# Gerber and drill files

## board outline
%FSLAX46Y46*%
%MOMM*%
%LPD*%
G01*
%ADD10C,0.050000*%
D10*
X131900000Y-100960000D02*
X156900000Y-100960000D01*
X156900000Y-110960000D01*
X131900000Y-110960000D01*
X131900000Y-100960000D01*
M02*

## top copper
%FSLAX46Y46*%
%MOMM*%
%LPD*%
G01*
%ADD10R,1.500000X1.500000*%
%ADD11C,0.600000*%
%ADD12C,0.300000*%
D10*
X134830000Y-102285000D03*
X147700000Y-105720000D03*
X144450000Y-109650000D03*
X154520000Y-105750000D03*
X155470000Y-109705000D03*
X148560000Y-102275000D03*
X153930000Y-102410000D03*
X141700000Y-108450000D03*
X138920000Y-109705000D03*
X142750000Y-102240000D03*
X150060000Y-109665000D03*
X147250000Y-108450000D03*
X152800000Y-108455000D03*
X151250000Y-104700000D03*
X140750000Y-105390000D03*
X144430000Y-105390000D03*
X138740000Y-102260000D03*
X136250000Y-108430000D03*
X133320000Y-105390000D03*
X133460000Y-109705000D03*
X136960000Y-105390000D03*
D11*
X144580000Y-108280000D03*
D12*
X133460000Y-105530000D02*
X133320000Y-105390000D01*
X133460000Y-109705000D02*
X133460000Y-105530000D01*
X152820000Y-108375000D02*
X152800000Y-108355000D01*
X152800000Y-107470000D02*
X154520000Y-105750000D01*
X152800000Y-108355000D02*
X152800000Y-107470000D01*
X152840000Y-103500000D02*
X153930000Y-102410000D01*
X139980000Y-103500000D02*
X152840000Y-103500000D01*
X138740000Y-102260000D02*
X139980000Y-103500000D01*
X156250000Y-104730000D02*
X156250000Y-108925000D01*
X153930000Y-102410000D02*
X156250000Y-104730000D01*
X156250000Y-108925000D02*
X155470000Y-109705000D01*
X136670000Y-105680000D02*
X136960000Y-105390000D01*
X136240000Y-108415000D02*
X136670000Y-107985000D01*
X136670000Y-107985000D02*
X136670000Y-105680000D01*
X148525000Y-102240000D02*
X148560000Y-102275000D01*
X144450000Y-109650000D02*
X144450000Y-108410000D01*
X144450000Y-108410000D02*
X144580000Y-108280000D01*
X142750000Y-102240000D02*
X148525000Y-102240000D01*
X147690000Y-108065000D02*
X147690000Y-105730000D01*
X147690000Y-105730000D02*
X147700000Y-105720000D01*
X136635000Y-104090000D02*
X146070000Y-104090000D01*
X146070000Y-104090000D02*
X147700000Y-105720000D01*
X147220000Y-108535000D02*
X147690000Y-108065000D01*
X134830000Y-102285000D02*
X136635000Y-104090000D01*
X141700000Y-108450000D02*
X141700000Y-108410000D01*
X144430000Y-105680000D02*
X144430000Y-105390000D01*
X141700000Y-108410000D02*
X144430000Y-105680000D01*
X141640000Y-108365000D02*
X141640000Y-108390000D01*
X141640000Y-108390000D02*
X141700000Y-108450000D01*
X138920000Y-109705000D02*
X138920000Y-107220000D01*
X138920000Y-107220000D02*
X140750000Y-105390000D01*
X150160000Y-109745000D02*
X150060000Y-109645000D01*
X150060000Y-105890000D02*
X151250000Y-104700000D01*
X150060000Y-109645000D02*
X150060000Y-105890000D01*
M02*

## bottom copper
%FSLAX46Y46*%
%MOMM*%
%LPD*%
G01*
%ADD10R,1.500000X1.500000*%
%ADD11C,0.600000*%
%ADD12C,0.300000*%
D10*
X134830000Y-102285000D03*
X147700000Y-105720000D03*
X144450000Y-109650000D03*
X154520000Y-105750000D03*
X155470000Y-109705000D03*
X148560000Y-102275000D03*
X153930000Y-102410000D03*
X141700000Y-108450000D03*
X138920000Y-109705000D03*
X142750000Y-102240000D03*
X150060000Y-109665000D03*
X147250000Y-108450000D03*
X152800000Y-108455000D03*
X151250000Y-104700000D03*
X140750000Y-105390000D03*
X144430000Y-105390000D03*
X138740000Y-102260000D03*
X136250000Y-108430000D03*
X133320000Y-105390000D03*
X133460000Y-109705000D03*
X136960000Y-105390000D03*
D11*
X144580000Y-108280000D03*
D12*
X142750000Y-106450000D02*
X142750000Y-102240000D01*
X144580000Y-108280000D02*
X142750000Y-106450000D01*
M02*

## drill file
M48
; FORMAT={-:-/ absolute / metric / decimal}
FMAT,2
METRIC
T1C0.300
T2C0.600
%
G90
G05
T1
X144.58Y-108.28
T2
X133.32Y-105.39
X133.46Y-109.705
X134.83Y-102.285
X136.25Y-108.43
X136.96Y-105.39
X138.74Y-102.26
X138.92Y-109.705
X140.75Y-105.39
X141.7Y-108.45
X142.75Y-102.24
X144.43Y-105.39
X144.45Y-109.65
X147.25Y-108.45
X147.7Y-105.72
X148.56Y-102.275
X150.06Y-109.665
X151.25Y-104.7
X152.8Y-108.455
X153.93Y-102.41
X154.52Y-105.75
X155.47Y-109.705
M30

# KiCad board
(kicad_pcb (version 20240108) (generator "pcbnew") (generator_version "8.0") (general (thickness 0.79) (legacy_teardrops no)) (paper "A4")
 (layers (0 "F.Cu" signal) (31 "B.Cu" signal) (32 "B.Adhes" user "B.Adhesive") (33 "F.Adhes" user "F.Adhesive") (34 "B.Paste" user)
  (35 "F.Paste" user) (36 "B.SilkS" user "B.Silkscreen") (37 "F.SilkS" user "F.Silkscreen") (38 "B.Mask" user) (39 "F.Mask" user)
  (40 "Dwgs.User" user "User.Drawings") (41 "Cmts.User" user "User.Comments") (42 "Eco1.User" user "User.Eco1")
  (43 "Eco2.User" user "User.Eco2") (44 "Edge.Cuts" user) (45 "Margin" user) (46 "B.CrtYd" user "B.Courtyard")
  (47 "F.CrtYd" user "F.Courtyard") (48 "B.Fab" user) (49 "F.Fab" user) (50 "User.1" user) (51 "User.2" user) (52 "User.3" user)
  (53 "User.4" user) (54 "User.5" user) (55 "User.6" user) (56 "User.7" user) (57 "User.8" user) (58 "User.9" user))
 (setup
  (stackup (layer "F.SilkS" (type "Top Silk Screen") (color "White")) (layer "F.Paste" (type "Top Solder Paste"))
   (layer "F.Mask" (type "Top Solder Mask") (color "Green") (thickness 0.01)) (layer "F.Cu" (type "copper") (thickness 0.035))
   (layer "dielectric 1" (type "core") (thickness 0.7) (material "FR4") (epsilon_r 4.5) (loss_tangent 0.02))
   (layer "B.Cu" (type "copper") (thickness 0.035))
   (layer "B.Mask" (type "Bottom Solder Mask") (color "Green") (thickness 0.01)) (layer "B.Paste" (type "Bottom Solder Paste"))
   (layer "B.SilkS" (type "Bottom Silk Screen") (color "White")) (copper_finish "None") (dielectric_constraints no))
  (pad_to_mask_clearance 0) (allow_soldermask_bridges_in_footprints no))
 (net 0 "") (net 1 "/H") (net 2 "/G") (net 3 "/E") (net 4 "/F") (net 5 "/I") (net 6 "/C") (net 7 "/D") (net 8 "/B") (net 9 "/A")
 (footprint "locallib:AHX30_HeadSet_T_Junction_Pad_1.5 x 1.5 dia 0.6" (layer "F.Cu") (at 134.83 102.285 180)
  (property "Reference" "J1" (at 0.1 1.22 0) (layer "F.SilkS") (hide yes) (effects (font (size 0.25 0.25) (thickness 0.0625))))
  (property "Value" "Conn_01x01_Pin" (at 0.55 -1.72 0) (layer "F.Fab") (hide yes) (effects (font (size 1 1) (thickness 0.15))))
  (pad "1" thru_hole rect (at 0 0 180) (size 1.5 1.5) (drill 0.6) (layers "*.Cu" "*.Mask") (remove_unused_layers no) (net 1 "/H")))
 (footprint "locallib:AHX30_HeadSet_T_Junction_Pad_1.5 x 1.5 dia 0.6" (layer "F.Cu") (at 147.7 105.72 180)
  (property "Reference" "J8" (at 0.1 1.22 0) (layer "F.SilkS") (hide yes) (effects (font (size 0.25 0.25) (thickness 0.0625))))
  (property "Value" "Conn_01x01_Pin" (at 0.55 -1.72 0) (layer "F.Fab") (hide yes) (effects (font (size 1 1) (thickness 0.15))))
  (pad "1" thru_hole rect (at 0 0 180) (size 1.5 1.5) (drill 0.6) (layers "*.Cu" "*.Mask") (remove_unused_layers no) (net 1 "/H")))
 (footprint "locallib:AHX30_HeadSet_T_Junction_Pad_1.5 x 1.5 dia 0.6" (layer "F.Cu") (at 144.45 109.65)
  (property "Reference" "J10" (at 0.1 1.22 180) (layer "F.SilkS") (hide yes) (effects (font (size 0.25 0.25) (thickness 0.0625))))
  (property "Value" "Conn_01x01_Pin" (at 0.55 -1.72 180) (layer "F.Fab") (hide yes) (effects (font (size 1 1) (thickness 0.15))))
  (pad "1" thru_hole rect (at 0 0) (size 1.5 1.5) (drill 0.6) (layers "*.Cu" "*.Mask") (remove_unused_layers no) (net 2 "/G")))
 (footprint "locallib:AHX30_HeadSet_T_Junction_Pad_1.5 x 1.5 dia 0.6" (layer "F.Cu") (at 154.52 105.75 180)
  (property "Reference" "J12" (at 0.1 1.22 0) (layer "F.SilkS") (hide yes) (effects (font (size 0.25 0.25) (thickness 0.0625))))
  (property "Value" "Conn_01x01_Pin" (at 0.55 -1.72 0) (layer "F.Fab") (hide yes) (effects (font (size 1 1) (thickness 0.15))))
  (pad "1" thru_hole rect (at 0 0 180) (size 1.5 1.5) (drill 0.6) (layers "*.Cu" "*.Mask") (remove_unused_layers no) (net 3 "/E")))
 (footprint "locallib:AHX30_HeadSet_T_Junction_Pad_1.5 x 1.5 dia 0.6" (layer "F.Cu") (at 155.47 109.705)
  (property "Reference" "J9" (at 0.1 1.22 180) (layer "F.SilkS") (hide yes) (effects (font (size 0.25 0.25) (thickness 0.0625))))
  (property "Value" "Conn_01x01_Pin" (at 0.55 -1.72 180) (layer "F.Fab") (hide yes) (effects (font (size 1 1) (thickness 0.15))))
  (pad "1" thru_hole rect (at 0 0) (size 1.5 1.5) (drill 0.6) (layers "*.Cu" "*.Mask") (remove_unused_layers no) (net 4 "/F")))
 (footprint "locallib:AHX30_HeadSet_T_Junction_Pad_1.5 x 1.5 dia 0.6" (layer "F.Cu") (at 148.56 102.275)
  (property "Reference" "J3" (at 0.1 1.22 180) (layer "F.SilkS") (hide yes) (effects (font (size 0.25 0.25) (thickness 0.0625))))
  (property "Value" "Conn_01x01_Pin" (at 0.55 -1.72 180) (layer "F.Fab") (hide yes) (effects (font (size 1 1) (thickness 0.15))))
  (pad "1" thru_hole rect (at 0 0) (size 1.5 1.5) (drill 0.6) (layers "*.Cu" "*.Mask") (remove_unused_layers no) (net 2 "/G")))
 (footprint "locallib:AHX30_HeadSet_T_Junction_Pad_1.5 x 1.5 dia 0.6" (layer "F.Cu") (at 153.93 102.41 180)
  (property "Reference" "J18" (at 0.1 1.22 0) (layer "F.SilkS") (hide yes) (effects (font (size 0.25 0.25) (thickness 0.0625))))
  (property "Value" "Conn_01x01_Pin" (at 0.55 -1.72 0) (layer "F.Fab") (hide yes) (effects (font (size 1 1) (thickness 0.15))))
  (pad "1" thru_hole rect (at 0 0 180) (size 1.5 1.5) (drill 0.6) (layers "*.Cu" "*.Mask") (remove_unused_layers no) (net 4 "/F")))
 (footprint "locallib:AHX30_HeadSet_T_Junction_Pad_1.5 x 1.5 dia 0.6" (layer "F.Cu") (at 141.7 108.45)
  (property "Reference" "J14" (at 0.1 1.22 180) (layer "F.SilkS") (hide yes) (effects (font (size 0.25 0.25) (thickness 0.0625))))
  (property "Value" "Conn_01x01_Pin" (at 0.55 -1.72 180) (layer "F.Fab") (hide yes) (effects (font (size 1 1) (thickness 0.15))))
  (pad "1" thru_hole rect (at 0 0) (size 1.5 1.5) (drill 0.6) (layers "*.Cu" "*.Mask") (remove_unused_layers no) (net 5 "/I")))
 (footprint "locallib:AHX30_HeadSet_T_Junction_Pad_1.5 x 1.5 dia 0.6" (layer "F.Cu") (at 138.92 109.705)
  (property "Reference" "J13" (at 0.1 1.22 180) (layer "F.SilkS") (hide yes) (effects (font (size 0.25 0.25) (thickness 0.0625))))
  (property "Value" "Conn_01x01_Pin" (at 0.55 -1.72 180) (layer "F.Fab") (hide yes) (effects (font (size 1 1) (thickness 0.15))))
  (pad "1" thru_hole rect (at 0 0) (size 1.5 1.5) (drill 0.6) (layers "*.Cu" "*.Mask") (remove_unused_layers no) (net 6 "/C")))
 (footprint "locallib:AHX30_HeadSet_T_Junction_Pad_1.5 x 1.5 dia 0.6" (layer "F.Cu") (at 142.75 102.24 180)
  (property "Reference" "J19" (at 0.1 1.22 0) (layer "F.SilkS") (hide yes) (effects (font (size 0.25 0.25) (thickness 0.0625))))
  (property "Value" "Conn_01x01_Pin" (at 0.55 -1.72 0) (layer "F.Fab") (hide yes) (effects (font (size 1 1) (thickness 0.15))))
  (pad "1" thru_hole rect (at 0 0 180) (size 1.5 1.5) (drill 0.6) (layers "*.Cu" "*.Mask") (remove_unused_layers no) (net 2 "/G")))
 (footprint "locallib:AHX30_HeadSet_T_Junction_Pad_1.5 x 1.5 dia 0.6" (layer "F.Cu") (at 150.06 109.665)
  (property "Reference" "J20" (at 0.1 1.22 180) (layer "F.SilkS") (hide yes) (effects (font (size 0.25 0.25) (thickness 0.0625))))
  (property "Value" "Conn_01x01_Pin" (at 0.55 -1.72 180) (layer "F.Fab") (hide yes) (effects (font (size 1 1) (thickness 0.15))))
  (pad "1" thru_hole rect (at 0 0) (size 1.5 1.5) (drill 0.6) (layers "*.Cu" "*.Mask") (remove_unused_layers no) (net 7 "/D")))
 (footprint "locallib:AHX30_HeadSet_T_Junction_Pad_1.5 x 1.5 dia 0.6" (layer "F.Cu") (at 147.25 108.45)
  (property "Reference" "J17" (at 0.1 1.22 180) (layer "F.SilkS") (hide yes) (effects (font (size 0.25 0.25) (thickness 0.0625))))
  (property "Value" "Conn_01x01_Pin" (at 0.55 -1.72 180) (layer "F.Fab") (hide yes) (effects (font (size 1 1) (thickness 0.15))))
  (pad "1" thru_hole rect (at 0 0) (size 1.5 1.5) (drill 0.6) (layers "*.Cu" "*.Mask") (remove_unused_layers no) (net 1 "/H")))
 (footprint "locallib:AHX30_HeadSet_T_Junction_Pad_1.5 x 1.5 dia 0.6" (layer "F.Cu") (at 152.8 108.455)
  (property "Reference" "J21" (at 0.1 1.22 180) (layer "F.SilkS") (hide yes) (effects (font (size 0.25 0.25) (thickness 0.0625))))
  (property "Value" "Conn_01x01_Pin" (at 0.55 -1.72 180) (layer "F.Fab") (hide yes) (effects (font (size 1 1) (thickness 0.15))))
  (pad "1" thru_hole rect (at 0 0) (size 1.5 1.5) (drill 0.6) (layers "*.Cu" "*.Mask") (remove_unused_layers no) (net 3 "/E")))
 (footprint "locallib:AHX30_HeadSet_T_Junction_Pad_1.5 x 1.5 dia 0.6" (layer "F.Cu") (at 151.25 104.7 180)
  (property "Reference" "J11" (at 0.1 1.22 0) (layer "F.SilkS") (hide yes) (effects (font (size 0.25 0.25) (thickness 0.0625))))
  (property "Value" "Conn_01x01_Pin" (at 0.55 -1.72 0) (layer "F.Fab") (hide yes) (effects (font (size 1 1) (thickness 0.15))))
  (pad "1" thru_hole rect (at 0 0 180) (size 1.5 1.5) (drill 0.6) (layers "*.Cu" "*.Mask") (remove_unused_layers no) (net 7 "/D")))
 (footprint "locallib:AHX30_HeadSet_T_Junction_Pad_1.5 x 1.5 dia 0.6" (layer "F.Cu") (at 140.75 105.39 180)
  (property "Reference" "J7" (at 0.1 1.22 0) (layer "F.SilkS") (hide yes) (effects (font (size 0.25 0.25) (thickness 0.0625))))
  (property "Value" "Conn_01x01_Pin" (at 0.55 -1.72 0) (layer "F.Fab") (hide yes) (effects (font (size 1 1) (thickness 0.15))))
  (pad "1" thru_hole rect (at 0 0 180) (size 1.5 1.5) (drill 0.6) (layers "*.Cu" "*.Mask") (remove_unused_layers no) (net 6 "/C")))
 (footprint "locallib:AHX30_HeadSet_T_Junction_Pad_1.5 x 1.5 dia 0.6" (layer "F.Cu") (at 144.43 105.39 180)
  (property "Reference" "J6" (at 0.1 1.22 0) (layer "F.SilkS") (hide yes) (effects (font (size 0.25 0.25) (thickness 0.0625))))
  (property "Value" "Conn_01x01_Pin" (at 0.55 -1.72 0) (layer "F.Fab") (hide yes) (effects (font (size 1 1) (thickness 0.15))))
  (pad "1" thru_hole rect (at 0 0 180) (size 1.5 1.5) (drill 0.6) (layers "*.Cu" "*.Mask") (remove_unused_layers no) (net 5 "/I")))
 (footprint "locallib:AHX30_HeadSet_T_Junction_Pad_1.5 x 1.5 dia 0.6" (layer "F.Cu") (at 138.74 102.26 180)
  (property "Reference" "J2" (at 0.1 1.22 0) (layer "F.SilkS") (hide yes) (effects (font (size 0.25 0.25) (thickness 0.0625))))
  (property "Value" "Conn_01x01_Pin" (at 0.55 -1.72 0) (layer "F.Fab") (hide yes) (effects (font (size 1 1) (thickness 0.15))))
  (pad "1" thru_hole rect (at 0 0 180) (size 1.5 1.5) (drill 0.6) (layers "*.Cu" "*.Mask") (remove_unused_layers no) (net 4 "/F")))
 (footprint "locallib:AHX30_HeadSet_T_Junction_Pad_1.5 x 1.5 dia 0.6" (layer "F.Cu") (at 136.25 108.43)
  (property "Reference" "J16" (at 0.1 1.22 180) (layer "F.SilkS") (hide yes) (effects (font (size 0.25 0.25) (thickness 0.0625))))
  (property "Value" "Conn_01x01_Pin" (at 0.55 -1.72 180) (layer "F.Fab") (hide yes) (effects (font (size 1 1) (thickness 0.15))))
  (pad "1" thru_hole rect (at 0 0) (size 1.5 1.5) (drill 0.6) (layers "*.Cu" "*.Mask") (remove_unused_layers no) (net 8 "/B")))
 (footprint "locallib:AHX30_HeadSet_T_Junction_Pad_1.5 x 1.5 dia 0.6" (layer "F.Cu") (at 133.32 105.39 180)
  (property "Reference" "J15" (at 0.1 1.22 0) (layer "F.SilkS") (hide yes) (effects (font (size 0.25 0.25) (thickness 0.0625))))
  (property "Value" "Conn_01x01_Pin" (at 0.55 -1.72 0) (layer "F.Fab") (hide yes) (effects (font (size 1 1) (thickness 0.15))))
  (pad "1" thru_hole rect (at 0 0 180) (size 1.5 1.5) (drill 0.6) (layers "*.Cu" "*.Mask") (remove_unused_layers no) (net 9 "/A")))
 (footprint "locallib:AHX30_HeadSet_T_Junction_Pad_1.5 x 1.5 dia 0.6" (layer "F.Cu") (at 133.46 109.705)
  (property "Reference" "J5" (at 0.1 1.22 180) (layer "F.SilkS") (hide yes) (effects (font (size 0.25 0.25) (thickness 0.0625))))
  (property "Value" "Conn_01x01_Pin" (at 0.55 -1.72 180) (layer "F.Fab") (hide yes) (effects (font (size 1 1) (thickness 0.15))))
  (pad "1" thru_hole rect (at 0 0) (size 1.5 1.5) (drill 0.6) (layers "*.Cu" "*.Mask") (remove_unused_layers no) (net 9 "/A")))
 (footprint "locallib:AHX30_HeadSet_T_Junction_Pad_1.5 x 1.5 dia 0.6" (layer "F.Cu") (at 136.96 105.39 180)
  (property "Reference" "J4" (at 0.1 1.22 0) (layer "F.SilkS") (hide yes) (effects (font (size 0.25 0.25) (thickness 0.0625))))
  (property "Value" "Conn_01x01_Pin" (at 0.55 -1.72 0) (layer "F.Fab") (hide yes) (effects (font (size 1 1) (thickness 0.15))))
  (pad "1" thru_hole rect (at 0 0 180) (size 1.5 1.5) (drill 0.6) (layers "*.Cu" "*.Mask") (remove_unused_layers no) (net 8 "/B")))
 (gr_rect (start 131.9 100.96) (end 156.9 110.96) (stroke (width 0.05) (type default)) (fill none) (layer "Edge.Cuts"))
 (segment (start 133.46 105.53) (end 133.32 105.39) (width 0.3) (layer "F.Cu") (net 9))
 (segment (start 133.46 109.705) (end 133.46 105.53) (width 0.3) (layer "F.Cu") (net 9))
 (segment (start 152.82 108.375) (end 152.8 108.355) (width 0.3) (layer "F.Cu") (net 3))
 (segment (start 152.8 107.47) (end 154.52 105.75) (width 0.3) (layer "F.Cu") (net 3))
 (segment (start 152.8 108.355) (end 152.8 107.47) (width 0.3) (layer "F.Cu") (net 3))
 (segment (start 152.84 103.5) (end 153.93 102.41) (width 0.3) (layer "F.Cu") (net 4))
 (segment (start 139.98 103.5) (end 152.84 103.5) (width 0.3) (layer "F.Cu") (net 4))
 (segment (start 138.74 102.26) (end 139.98 103.5) (width 0.3) (layer "F.Cu") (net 4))
 (segment (start 156.25 104.73) (end 156.25 108.925) (width 0.3) (layer "F.Cu") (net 4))
 (segment (start 153.93 102.41) (end 156.25 104.73) (width 0.3) (layer "F.Cu") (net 4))
 (segment (start 156.25 108.925) (end 155.47 109.705) (width 0.3) (layer "F.Cu") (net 4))
 (segment (start 136.67 105.68) (end 136.96 105.39) (width 0.3) (layer "F.Cu") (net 8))
 (segment (start 136.24 108.415) (end 136.67 107.985) (width 0.3) (layer "F.Cu") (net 8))
 (segment (start 136.67 107.985) (end 136.67 105.68) (width 0.3) (layer "F.Cu") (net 8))
 (segment (start 148.525 102.24) (end 148.56 102.275) (width 0.3) (layer "F.Cu") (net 2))
 (segment (start 144.45 109.65) (end 144.45 108.41) (width 0.3) (layer "F.Cu") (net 2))
 (segment (start 144.45 108.41) (end 144.58 108.28) (width 0.3) (layer "F.Cu") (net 2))
 (segment (start 142.75 102.24) (end 148.525 102.24) (width 0.3) (layer "F.Cu") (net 2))
 (via (at 144.58 108.28) (size 0.6) (drill 0.3) (layers "F.Cu" "B.Cu") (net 2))
 (segment (start 142.75 106.45) (end 142.75 102.24) (width 0.3) (layer "B.Cu") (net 2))
 (segment (start 144.58 108.28) (end 142.75 106.45) (width 0.3) (layer "B.Cu") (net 2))
 (segment (start 147.69 108.065) (end 147.69 105.73) (width 0.3) (layer "F.Cu") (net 1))
 (segment (start 147.69 105.73) (end 147.7 105.72) (width 0.3) (layer "F.Cu") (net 1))
 (segment (start 136.635 104.09) (end 146.07 104.09) (width 0.3) (layer "F.Cu") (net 1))
 (segment (start 146.07 104.09) (end 147.7 105.72) (width 0.3) (layer "F.Cu") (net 1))
 (segment (start 147.22 108.535) (end 147.69 108.065) (width 0.3) (layer "F.Cu") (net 1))
 (segment (start 134.83 102.285) (end 136.635 104.09) (width 0.3) (layer "F.Cu") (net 1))
 (segment (start 141.7 108.45) (end 141.7 108.41) (width 0.3) (layer "F.Cu") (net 5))
 (segment (start 144.43 105.68) (end 144.43 105.39) (width 0.3) (layer "F.Cu") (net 5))
 (segment (start 141.7 108.41) (end 144.43 105.68) (width 0.3) (layer "F.Cu") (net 5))
 (segment (start 141.64 108.365) (end 141.64 108.39) (width 0.3) (layer "F.Cu") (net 5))
 (segment (start 141.64 108.39) (end 141.7 108.45) (width 0.3) (layer "F.Cu") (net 5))
 (segment (start 138.92 109.705) (end 138.92 107.22) (width 0.3) (layer "F.Cu") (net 6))
 (segment (start 138.92 107.22) (end 140.75 105.39) (width 0.3) (layer "F.Cu") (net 6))
 (segment (start 150.16 109.745) (end 150.06 109.645) (width 0.3) (layer "F.Cu") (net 7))
 (segment (start 150.06 105.89) (end 151.25 104.7) (width 0.3) (layer "F.Cu") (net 7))
 (segment (start 150.06 109.645) (end 150.06 105.89) (width 0.3) (layer "F.Cu") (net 7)))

